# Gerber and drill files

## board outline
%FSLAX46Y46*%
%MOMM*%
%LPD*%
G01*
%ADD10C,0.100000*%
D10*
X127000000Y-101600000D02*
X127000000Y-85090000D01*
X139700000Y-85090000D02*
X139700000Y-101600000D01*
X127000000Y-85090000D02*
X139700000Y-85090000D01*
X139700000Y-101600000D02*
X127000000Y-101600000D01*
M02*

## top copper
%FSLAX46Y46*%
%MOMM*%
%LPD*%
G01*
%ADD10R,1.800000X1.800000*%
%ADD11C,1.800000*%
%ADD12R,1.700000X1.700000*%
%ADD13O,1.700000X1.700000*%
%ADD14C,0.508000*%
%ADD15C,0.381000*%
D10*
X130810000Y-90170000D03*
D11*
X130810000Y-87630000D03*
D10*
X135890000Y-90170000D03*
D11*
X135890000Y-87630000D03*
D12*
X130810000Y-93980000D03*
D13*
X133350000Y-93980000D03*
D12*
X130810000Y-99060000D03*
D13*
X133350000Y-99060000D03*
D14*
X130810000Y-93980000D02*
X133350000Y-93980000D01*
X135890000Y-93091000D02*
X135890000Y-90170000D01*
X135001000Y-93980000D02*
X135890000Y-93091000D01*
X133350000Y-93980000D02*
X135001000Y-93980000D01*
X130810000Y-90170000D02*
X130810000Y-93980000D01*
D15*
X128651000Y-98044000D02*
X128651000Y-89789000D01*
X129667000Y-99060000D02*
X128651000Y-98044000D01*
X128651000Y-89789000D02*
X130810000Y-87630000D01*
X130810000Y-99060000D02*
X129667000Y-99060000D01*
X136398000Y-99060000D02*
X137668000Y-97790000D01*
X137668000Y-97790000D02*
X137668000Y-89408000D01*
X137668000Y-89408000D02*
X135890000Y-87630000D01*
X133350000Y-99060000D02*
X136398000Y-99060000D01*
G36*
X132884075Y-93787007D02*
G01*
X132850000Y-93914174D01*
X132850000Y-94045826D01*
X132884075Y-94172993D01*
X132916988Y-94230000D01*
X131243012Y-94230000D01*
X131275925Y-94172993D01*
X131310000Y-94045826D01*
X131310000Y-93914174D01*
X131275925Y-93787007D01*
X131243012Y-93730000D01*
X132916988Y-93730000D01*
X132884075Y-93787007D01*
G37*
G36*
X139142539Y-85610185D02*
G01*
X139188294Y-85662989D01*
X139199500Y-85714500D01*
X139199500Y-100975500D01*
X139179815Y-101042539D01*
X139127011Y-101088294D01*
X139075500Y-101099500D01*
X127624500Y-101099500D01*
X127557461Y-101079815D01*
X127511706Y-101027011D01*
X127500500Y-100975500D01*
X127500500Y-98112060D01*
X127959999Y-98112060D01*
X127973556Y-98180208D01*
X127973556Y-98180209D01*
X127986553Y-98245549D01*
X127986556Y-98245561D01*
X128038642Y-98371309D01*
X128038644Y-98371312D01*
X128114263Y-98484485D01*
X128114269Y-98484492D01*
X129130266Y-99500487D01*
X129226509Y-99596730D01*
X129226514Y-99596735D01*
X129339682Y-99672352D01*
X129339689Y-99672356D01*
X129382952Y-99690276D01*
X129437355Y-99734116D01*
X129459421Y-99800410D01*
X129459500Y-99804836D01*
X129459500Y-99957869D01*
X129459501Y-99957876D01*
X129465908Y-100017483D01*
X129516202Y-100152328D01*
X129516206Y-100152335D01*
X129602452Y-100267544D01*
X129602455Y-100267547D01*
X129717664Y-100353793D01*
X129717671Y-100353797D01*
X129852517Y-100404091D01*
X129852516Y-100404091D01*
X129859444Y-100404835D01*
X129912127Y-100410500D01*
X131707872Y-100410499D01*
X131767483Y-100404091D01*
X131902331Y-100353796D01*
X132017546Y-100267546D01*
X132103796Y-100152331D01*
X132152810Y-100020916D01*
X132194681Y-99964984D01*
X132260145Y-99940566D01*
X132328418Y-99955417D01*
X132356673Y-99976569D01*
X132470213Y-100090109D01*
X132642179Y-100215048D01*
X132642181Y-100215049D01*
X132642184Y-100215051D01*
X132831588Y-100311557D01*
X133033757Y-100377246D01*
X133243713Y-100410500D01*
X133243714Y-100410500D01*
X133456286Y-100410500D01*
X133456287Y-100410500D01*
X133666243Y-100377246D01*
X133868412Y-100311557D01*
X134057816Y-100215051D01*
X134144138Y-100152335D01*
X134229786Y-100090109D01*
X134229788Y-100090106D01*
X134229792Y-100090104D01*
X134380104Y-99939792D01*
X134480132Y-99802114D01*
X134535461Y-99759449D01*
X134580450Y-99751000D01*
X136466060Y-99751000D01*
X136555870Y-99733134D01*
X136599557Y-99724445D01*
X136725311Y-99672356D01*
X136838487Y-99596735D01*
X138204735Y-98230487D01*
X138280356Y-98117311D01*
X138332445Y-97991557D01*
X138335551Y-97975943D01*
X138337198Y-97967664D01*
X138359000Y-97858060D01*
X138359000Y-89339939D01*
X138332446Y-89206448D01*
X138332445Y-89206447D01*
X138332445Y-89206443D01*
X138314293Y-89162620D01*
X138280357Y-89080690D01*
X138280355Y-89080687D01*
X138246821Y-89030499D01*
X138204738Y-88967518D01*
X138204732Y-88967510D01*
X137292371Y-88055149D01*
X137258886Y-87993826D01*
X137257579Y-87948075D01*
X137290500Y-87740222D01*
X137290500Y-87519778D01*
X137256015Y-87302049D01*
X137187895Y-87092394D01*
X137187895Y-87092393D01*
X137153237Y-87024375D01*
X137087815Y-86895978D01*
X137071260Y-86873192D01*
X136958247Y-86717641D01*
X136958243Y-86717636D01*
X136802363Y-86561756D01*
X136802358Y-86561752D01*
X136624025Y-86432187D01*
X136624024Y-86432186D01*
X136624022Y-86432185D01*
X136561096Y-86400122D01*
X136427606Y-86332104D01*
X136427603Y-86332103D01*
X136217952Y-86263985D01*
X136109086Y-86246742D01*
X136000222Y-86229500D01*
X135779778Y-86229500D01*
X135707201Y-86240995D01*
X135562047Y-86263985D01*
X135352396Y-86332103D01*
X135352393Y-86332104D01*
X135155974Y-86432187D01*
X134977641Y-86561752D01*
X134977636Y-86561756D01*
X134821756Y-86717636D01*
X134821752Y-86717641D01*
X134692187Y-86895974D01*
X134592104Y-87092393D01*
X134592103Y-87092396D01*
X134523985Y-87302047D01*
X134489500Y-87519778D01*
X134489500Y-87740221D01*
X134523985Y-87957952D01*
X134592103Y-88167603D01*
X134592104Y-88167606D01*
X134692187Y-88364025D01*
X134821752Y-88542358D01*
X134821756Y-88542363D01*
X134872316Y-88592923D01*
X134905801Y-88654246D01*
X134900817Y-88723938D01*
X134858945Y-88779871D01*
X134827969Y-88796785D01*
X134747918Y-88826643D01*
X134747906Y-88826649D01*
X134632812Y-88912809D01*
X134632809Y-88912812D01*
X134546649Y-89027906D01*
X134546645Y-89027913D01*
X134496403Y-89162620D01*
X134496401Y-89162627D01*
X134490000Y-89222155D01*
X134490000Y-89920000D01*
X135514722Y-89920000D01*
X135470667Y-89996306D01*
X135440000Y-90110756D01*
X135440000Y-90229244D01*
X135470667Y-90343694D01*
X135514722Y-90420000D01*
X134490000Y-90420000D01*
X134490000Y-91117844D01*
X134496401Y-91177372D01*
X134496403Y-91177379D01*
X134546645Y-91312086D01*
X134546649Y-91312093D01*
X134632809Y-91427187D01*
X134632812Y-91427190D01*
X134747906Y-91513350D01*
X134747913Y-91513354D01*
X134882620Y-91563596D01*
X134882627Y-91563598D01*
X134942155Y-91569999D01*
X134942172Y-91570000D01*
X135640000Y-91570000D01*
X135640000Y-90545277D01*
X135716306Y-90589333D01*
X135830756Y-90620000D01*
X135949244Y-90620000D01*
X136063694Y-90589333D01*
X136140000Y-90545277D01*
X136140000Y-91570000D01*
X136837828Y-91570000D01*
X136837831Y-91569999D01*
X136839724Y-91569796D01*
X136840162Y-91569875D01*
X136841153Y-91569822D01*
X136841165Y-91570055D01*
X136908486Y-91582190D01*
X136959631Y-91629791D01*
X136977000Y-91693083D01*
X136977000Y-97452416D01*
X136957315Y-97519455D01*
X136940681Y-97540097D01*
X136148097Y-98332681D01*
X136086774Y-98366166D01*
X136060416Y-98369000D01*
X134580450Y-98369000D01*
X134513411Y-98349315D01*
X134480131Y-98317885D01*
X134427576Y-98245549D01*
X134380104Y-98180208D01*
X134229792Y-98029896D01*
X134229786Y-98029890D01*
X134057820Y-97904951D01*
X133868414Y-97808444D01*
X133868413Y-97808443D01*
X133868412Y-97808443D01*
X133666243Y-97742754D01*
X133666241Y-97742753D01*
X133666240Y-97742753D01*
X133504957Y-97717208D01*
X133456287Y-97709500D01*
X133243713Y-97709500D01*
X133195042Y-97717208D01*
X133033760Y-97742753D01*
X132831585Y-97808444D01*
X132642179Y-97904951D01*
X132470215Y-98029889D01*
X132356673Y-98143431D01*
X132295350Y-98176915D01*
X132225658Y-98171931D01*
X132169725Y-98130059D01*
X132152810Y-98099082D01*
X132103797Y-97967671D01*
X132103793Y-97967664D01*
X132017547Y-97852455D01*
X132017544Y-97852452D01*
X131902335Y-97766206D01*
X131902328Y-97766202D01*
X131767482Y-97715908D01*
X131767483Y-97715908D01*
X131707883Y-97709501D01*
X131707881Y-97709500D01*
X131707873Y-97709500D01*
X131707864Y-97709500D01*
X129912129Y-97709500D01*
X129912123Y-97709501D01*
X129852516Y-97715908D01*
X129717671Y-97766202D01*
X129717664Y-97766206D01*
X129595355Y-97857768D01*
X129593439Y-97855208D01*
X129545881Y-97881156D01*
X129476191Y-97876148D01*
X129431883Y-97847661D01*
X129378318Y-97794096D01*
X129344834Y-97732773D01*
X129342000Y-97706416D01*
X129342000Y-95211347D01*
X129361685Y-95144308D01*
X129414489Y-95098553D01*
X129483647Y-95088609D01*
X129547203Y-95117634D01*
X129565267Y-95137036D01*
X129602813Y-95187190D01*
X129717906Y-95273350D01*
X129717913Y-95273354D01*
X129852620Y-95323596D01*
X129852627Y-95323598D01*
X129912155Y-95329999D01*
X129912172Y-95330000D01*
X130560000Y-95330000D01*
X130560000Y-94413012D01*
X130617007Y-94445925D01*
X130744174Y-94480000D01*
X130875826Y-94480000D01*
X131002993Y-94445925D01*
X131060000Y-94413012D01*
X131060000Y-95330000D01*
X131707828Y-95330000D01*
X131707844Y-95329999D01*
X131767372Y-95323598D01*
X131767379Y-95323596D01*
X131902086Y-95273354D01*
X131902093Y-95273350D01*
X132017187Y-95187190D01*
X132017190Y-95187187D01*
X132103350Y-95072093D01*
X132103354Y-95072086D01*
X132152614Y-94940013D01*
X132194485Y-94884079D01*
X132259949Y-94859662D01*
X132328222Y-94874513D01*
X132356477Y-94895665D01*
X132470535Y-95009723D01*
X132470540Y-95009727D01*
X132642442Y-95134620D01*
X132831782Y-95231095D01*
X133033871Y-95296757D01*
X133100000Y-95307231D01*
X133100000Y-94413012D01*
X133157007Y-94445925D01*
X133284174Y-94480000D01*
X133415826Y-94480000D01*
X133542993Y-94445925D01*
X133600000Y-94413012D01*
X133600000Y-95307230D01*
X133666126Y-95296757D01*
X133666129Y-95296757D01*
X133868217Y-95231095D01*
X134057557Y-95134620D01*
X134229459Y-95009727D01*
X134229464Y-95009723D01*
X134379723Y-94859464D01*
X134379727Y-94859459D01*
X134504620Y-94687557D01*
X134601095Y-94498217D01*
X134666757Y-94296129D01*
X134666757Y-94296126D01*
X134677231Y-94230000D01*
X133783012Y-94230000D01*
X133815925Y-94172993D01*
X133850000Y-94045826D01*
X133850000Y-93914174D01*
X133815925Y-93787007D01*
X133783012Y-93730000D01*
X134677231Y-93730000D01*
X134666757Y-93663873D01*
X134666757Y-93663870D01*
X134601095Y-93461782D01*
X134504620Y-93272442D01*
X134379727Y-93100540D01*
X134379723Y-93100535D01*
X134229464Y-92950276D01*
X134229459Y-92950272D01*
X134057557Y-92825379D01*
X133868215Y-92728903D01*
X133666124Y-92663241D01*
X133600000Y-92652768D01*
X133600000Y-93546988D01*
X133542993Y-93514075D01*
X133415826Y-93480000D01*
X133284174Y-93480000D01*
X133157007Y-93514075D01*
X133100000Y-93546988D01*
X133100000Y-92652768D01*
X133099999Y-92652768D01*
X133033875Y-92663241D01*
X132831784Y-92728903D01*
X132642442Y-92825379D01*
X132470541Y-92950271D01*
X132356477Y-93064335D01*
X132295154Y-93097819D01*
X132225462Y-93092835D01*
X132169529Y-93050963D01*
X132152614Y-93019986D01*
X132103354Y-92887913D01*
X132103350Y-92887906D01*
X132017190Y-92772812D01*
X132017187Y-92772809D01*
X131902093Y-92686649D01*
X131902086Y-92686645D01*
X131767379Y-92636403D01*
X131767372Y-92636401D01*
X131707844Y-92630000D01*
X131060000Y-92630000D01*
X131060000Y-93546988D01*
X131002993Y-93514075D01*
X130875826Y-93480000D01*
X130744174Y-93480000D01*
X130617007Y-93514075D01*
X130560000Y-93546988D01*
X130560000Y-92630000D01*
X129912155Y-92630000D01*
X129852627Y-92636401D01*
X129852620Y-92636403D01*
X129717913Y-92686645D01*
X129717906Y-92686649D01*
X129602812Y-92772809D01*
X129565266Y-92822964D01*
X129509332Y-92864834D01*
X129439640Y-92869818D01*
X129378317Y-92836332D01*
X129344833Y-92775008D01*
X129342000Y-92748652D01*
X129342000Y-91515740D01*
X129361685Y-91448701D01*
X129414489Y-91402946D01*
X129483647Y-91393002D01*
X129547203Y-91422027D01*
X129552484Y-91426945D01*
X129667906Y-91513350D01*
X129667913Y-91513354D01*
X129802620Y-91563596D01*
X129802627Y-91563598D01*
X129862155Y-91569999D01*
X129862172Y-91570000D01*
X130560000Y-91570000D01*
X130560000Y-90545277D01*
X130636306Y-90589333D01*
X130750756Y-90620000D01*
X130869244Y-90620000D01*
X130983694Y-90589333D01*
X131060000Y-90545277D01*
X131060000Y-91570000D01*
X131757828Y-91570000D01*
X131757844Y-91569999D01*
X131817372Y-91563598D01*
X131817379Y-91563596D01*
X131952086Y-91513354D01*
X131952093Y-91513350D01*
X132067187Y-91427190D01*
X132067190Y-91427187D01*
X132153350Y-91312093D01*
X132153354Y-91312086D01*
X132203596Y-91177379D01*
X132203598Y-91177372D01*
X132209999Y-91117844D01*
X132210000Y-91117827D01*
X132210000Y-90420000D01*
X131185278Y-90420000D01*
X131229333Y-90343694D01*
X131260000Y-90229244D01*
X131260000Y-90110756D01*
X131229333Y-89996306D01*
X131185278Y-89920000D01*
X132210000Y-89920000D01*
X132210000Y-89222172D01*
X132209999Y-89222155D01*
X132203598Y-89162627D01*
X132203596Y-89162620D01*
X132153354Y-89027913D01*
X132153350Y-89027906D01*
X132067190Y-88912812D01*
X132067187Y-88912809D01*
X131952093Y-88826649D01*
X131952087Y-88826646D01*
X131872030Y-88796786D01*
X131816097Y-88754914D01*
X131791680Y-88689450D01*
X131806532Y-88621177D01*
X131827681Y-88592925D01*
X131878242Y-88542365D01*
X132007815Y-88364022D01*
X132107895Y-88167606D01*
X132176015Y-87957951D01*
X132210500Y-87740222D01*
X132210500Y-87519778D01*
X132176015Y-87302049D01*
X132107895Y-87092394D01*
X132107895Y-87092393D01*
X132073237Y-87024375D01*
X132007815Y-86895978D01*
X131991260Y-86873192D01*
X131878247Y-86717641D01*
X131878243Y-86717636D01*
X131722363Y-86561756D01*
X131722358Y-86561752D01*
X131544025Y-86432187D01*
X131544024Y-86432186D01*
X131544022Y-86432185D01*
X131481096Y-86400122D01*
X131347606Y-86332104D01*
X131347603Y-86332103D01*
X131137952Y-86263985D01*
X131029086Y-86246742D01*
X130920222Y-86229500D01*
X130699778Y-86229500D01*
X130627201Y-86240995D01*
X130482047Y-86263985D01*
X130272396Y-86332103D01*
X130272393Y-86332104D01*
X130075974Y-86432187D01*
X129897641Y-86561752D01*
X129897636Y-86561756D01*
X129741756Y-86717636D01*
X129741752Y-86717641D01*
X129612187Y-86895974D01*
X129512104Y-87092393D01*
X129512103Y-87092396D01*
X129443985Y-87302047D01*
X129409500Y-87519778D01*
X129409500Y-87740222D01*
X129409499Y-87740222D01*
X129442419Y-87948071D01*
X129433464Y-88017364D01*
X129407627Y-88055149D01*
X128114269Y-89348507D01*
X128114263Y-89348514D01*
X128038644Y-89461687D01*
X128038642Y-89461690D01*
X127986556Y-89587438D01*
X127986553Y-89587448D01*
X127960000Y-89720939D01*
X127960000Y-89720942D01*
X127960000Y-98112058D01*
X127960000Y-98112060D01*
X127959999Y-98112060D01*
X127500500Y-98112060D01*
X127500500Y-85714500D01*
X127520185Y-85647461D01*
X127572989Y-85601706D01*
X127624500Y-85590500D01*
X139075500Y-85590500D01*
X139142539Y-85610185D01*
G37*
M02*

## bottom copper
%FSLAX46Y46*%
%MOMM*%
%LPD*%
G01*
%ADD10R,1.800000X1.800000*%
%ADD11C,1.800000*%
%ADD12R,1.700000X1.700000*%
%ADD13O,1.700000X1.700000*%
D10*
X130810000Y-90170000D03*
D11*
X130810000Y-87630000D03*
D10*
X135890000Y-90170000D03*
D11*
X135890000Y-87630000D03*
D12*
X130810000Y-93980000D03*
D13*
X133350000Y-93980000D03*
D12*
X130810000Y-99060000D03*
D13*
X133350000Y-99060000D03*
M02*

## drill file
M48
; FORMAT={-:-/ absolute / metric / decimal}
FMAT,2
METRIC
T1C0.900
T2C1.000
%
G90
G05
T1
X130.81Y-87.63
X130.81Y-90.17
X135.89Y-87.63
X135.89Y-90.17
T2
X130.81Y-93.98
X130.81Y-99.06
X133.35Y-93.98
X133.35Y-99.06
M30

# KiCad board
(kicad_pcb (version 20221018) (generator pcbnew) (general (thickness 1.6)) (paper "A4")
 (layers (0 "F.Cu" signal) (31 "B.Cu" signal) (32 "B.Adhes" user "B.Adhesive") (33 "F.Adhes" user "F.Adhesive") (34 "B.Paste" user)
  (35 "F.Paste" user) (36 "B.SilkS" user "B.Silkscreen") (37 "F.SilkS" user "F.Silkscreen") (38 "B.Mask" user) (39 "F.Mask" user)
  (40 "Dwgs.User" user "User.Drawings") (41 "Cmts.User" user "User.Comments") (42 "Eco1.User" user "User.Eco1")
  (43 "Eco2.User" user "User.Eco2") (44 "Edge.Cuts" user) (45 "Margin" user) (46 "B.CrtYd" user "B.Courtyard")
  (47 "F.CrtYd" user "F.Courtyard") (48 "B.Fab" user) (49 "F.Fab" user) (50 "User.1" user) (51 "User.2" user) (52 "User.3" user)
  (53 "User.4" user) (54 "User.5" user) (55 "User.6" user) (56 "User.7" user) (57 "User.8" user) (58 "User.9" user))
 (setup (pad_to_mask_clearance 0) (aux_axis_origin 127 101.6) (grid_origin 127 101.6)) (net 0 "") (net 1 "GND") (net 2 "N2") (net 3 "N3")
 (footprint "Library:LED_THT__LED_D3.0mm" (layer "F.Cu") (at 130.81 90.17 90)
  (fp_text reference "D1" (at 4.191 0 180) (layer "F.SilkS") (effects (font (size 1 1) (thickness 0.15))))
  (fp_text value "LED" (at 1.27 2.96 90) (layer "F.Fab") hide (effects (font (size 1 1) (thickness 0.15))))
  (pad "1" thru_hole rect (at 0 0 90) (size 1.8 1.8) (drill 0.9) (layers "*.Cu" "*.Mask") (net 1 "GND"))
  (pad "2" thru_hole circle (at 2.54 0 90) (size 1.8 1.8) (drill 0.9) (layers "*.Cu" "*.Mask") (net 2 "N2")))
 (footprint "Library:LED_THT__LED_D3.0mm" (layer "F.Cu") (at 135.89 90.17 90)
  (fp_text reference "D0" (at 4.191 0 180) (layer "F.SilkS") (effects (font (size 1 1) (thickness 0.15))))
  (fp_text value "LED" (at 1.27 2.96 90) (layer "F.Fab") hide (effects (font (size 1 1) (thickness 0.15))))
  (pad "1" thru_hole rect (at 0 0 90) (size 1.8 1.8) (drill 0.9) (layers "*.Cu" "*.Mask") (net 1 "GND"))
  (pad "2" thru_hole circle (at 2.54 0 90) (size 1.8 1.8) (drill 0.9) (layers "*.Cu" "*.Mask") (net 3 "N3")))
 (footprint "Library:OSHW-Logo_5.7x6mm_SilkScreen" (layer "F.Cu") (at 136.906 96.52)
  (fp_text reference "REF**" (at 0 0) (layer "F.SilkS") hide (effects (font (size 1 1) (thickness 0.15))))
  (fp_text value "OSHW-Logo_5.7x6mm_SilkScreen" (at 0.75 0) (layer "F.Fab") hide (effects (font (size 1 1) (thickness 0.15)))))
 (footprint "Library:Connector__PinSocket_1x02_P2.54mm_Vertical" (layer "B.Cu") (at 130.81 93.98 -90)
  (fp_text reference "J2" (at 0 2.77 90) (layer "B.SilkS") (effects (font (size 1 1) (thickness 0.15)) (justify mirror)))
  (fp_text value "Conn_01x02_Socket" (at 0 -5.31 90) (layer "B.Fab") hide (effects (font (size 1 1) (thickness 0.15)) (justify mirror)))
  (pad "1" thru_hole rect (at 0 0 270) (size 1.7 1.7) (drill 1) (layers "*.Cu" "*.Mask") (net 1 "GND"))
  (pad "2" thru_hole oval (at 0 -2.54 270) (size 1.7 1.7) (drill 1) (layers "*.Cu" "*.Mask") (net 1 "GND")))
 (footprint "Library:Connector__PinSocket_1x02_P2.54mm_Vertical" (layer "B.Cu") (at 130.81 99.06 -90)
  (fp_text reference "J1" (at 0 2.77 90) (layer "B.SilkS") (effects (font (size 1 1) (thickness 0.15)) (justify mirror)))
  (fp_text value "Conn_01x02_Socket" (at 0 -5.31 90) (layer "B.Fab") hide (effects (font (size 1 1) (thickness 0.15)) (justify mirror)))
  (pad "1" thru_hole rect (at 0 0 270) (size 1.7 1.7) (drill 1) (layers "*.Cu" "*.Mask") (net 2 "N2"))
  (pad "2" thru_hole oval (at 0 -2.54 270) (size 1.7 1.7) (drill 1) (layers "*.Cu" "*.Mask") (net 3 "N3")))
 (gr_line (start 127 101.6) (end 127 85.09) (stroke (width 0.1) (type default)) (layer "Edge.Cuts"))
 (gr_line (start 139.7 85.09) (end 139.7 101.6) (stroke (width 0.1) (type default)) (layer "Edge.Cuts"))
 (gr_line (start 127 85.09) (end 139.7 85.09) (stroke (width 0.1) (type default)) (layer "Edge.Cuts"))
 (gr_line (start 139.7 101.6) (end 127 101.6) (stroke (width 0.1) (type default)) (layer "Edge.Cuts"))
 (segment (start 130.81 93.98) (end 133.35 93.98) (width 0.508) (layer "F.Cu") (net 1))
 (segment (start 135.89 93.091) (end 135.89 90.17) (width 0.508) (layer "F.Cu") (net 1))
 (segment (start 135.001 93.98) (end 135.89 93.091) (width 0.508) (layer "F.Cu") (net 1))
 (segment (start 133.35 93.98) (end 135.001 93.98) (width 0.508) (layer "F.Cu") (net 1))
 (segment (start 130.81 90.17) (end 130.81 93.98) (width 0.508) (layer "F.Cu") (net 1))
 (segment (start 128.651 98.044) (end 128.651 89.789) (width 0.381) (layer "F.Cu") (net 2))
 (segment (start 129.667 99.06) (end 128.651 98.044) (width 0.381) (layer "F.Cu") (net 2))
 (segment (start 128.651 89.789) (end 130.81 87.63) (width 0.381) (layer "F.Cu") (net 2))
 (segment (start 130.81 99.06) (end 129.667 99.06) (width 0.381) (layer "F.Cu") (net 2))
 (segment (start 136.398 99.06) (end 137.668 97.79) (width 0.381) (layer "F.Cu") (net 3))
 (segment (start 137.668 97.79) (end 137.668 89.408) (width 0.381) (layer "F.Cu") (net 3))
 (segment (start 137.668 89.408) (end 135.89 87.63) (width 0.381) (layer "F.Cu") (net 3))
 (segment (start 133.35 99.06) (end 136.398 99.06) (width 0.381) (layer "F.Cu") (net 3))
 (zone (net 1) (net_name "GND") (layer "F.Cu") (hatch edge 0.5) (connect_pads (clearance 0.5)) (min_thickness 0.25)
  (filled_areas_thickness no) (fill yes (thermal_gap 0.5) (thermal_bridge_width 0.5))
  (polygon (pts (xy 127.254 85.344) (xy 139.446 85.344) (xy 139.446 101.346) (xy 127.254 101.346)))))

